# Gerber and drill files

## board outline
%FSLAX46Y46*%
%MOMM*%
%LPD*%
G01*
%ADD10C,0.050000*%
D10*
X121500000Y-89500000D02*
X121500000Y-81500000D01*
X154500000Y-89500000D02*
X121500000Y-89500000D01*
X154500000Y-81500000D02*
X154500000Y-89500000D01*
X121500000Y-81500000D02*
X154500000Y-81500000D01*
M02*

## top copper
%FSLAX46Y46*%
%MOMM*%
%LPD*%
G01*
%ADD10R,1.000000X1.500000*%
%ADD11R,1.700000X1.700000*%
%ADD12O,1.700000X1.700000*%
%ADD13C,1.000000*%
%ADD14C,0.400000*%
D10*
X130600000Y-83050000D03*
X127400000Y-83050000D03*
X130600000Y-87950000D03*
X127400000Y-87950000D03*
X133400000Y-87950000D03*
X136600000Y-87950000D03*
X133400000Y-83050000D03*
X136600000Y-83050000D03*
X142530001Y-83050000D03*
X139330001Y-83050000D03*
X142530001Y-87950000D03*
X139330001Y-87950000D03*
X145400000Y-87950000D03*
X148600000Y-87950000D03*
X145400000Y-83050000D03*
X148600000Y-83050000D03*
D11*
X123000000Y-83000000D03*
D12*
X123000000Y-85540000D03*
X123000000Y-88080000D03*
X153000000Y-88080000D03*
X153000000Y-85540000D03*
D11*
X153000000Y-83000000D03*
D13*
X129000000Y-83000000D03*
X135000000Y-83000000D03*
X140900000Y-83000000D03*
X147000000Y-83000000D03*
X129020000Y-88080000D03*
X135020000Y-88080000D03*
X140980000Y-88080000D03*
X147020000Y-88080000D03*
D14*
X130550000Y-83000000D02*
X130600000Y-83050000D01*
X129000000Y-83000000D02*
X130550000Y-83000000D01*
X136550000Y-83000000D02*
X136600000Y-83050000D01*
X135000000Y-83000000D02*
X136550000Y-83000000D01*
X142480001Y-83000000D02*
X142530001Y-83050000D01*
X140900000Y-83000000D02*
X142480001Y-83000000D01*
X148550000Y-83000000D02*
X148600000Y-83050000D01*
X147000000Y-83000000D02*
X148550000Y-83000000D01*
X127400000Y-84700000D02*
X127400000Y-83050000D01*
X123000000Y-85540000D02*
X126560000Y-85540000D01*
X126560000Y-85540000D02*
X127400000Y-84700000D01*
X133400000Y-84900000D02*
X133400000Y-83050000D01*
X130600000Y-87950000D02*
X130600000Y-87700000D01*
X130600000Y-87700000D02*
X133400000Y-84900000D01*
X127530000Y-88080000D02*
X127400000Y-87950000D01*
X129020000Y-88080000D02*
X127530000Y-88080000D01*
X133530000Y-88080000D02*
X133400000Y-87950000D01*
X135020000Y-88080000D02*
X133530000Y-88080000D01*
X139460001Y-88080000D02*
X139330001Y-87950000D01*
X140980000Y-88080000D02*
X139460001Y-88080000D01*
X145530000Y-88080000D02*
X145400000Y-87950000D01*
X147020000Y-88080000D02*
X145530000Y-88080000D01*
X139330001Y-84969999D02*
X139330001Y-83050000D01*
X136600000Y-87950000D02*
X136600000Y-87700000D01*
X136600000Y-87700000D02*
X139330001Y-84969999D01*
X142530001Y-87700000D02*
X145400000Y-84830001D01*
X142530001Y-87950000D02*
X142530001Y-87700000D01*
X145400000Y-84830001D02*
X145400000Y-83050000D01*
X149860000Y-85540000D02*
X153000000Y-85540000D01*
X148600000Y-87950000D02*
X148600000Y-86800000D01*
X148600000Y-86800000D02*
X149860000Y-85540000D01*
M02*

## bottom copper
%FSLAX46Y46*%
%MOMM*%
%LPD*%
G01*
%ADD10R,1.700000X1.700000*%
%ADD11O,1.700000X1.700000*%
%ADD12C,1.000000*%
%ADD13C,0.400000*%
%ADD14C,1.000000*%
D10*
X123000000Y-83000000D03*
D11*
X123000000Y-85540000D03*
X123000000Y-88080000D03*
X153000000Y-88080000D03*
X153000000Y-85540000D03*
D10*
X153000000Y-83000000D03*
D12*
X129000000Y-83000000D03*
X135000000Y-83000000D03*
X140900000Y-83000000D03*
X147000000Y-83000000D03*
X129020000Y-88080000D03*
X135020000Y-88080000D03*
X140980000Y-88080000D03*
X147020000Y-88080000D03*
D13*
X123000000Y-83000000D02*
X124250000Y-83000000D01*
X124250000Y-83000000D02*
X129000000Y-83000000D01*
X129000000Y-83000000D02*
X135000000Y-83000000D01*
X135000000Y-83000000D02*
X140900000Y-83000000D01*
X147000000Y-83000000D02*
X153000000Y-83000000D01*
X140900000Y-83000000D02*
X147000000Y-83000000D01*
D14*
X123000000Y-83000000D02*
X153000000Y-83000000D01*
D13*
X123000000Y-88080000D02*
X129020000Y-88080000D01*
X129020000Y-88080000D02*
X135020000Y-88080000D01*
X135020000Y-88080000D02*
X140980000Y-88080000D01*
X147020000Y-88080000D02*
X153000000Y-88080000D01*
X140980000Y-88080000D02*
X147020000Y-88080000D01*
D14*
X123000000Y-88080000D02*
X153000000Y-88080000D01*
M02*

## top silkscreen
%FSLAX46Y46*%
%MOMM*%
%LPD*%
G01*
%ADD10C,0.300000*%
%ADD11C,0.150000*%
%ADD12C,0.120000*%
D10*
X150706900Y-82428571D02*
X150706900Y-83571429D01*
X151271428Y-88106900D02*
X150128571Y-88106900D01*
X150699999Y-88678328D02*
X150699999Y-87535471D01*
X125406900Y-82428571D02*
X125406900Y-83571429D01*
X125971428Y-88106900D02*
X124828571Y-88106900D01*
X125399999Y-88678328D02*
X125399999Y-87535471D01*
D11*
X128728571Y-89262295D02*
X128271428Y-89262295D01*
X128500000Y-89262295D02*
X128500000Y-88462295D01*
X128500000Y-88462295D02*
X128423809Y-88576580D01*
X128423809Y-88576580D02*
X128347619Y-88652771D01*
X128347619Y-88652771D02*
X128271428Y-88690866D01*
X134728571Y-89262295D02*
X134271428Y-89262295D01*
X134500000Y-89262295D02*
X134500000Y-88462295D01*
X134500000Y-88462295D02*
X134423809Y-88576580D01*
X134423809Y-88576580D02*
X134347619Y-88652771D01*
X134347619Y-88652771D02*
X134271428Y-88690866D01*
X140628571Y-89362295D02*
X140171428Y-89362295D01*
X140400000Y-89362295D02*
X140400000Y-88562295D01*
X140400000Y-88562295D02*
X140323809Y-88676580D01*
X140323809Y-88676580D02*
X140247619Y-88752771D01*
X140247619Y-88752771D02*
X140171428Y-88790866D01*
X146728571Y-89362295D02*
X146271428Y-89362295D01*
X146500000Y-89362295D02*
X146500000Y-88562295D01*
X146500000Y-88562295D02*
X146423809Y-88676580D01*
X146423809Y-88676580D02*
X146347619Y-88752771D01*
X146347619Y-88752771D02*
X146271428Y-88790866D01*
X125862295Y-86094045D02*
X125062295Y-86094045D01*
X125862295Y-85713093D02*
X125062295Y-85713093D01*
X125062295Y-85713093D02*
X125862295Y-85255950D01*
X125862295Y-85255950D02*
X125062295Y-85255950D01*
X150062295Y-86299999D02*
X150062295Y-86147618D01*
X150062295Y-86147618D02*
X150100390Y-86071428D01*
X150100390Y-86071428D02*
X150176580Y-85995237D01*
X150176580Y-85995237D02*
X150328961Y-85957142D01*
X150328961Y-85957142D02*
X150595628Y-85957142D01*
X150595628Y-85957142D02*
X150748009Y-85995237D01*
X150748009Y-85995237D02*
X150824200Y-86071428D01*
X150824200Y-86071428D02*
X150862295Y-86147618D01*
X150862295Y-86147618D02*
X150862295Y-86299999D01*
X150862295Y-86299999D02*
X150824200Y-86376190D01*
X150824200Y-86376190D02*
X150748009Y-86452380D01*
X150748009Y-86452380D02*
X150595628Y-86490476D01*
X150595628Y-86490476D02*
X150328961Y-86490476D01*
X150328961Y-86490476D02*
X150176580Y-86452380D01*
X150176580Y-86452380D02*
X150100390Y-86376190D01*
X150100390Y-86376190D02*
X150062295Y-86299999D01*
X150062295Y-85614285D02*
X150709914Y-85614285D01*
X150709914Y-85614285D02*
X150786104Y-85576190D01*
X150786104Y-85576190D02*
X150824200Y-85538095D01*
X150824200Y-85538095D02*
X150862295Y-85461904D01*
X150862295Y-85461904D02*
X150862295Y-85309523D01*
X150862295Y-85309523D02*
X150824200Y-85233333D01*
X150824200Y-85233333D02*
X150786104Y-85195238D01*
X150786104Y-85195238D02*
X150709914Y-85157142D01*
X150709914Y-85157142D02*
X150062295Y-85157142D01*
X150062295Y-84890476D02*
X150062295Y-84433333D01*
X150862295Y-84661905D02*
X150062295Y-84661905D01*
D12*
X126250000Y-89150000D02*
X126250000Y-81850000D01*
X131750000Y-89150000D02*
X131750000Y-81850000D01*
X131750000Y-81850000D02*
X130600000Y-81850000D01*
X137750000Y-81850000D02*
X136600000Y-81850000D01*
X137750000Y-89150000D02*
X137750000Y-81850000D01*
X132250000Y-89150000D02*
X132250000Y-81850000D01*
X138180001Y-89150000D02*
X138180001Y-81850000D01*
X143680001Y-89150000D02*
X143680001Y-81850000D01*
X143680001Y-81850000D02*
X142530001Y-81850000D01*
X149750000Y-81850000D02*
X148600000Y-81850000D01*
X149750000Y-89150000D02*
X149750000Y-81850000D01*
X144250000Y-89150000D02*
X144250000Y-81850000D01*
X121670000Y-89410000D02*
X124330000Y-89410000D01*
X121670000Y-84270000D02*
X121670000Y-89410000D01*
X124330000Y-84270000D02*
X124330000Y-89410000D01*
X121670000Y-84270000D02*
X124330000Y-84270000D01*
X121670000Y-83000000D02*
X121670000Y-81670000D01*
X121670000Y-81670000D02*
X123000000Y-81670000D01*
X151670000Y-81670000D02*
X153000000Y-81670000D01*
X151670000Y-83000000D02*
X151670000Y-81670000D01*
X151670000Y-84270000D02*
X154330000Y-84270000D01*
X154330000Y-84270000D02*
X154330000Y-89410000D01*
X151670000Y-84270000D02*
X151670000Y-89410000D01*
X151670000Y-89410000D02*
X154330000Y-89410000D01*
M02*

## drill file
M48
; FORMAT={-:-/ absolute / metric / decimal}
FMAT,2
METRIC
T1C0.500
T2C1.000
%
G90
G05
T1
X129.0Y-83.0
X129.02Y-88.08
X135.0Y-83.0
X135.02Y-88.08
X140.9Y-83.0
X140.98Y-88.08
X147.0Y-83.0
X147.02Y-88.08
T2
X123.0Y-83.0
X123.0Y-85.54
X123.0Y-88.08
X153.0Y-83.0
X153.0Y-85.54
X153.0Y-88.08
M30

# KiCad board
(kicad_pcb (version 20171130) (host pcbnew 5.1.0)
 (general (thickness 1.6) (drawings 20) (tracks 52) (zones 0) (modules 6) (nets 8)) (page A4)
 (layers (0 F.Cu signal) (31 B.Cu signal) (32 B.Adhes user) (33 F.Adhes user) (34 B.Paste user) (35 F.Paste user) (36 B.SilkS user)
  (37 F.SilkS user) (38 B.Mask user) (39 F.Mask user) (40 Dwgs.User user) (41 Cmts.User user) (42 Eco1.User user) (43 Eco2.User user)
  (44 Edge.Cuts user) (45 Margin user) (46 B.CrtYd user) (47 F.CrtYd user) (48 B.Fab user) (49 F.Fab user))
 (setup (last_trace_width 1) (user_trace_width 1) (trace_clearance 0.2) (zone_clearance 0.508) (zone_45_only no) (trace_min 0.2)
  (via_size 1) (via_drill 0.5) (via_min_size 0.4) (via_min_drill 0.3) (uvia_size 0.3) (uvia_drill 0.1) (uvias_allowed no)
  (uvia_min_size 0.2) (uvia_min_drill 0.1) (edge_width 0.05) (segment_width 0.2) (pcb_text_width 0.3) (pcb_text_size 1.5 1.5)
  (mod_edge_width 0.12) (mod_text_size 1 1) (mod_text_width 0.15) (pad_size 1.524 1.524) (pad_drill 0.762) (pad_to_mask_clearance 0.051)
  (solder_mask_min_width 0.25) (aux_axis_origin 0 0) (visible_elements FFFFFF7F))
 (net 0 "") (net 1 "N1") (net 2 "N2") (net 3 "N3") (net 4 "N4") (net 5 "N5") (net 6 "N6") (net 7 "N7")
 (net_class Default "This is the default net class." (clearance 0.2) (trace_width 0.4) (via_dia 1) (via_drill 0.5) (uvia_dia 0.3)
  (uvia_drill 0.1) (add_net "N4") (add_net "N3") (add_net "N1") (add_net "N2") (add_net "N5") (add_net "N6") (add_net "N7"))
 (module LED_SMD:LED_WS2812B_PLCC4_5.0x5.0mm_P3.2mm (layer F.Cu) (at 129 85.5 90)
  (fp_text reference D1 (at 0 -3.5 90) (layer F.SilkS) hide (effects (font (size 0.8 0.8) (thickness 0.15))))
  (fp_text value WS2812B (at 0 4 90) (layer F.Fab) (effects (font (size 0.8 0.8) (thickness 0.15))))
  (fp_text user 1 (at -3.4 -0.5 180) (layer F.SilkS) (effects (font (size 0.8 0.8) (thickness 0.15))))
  (fp_line (start -3.65 -2.75) (end 3.65 -2.75) (layer F.SilkS) (width 0.12))
  (fp_line (start -3.65 2.75) (end 3.65 2.75) (layer F.SilkS) (width 0.12))
  (fp_line (start 3.65 2.75) (end 3.65 1.6) (layer F.SilkS) (width 0.12))
  (pad 3 smd rect (at 2.45 1.6 90) (size 1.5 1) (layers F.Cu F.Paste F.Mask) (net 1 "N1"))
  (pad 4 smd rect (at 2.45 -1.6 90) (size 1.5 1) (layers F.Cu F.Paste F.Mask) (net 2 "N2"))
  (pad 2 smd rect (at -2.45 1.6 90) (size 1.5 1) (layers F.Cu F.Paste F.Mask) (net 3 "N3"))
  (pad 1 smd rect (at -2.45 -1.6 90) (size 1.5 1) (layers F.Cu F.Paste F.Mask) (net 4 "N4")))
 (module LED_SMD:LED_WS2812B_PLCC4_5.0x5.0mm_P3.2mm (layer F.Cu) (at 135 85.5 90)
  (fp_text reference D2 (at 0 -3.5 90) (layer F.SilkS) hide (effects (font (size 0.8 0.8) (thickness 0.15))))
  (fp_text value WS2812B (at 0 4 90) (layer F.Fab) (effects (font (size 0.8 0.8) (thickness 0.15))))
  (fp_line (start 3.65 2.75) (end 3.65 1.6) (layer F.SilkS) (width 0.12))
  (fp_line (start -3.65 2.75) (end 3.65 2.75) (layer F.SilkS) (width 0.12))
  (fp_line (start -3.65 -2.75) (end 3.65 -2.75) (layer F.SilkS) (width 0.12))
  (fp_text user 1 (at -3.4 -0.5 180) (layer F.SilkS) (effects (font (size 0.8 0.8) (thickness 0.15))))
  (pad 1 smd rect (at -2.45 -1.6 90) (size 1.5 1) (layers F.Cu F.Paste F.Mask) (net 4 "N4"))
  (pad 2 smd rect (at -2.45 1.6 90) (size 1.5 1) (layers F.Cu F.Paste F.Mask) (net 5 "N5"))
  (pad 4 smd rect (at 2.45 -1.6 90) (size 1.5 1) (layers F.Cu F.Paste F.Mask) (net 3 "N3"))
  (pad 3 smd rect (at 2.45 1.6 90) (size 1.5 1) (layers F.Cu F.Paste F.Mask) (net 1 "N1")))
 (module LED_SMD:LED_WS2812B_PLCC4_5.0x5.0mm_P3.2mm (layer F.Cu) (at 140.930001 85.5 90)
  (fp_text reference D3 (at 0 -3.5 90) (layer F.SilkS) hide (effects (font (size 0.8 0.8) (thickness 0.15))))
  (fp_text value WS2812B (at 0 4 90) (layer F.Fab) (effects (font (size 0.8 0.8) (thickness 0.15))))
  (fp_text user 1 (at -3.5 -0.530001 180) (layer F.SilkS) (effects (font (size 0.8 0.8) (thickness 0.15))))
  (fp_line (start -3.65 -2.75) (end 3.65 -2.75) (layer F.SilkS) (width 0.12))
  (fp_line (start -3.65 2.75) (end 3.65 2.75) (layer F.SilkS) (width 0.12))
  (fp_line (start 3.65 2.75) (end 3.65 1.6) (layer F.SilkS) (width 0.12))
  (pad 3 smd rect (at 2.45 1.6 90) (size 1.5 1) (layers F.Cu F.Paste F.Mask) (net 1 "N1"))
  (pad 4 smd rect (at 2.45 -1.6 90) (size 1.5 1) (layers F.Cu F.Paste F.Mask) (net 5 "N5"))
  (pad 2 smd rect (at -2.45 1.6 90) (size 1.5 1) (layers F.Cu F.Paste F.Mask) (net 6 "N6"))
  (pad 1 smd rect (at -2.45 -1.6 90) (size 1.5 1) (layers F.Cu F.Paste F.Mask) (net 4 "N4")))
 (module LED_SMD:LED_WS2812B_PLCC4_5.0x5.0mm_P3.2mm (layer F.Cu) (at 147 85.5 90)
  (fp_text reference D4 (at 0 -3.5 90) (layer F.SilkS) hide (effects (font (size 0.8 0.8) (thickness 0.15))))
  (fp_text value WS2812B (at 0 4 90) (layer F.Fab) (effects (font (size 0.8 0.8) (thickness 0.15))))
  (fp_line (start 3.65 2.75) (end 3.65 1.6) (layer F.SilkS) (width 0.12))
  (fp_line (start -3.65 2.75) (end 3.65 2.75) (layer F.SilkS) (width 0.12))
  (fp_line (start -3.65 -2.75) (end 3.65 -2.75) (layer F.SilkS) (width 0.12))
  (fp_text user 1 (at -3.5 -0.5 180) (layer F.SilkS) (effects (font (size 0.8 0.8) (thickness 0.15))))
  (pad 1 smd rect (at -2.45 -1.6 90) (size 1.5 1) (layers F.Cu F.Paste F.Mask) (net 4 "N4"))
  (pad 2 smd rect (at -2.45 1.6 90) (size 1.5 1) (layers F.Cu F.Paste F.Mask) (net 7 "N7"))
  (pad 4 smd rect (at 2.45 -1.6 90) (size 1.5 1) (layers F.Cu F.Paste F.Mask) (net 6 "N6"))
  (pad 3 smd rect (at 2.45 1.6 90) (size 1.5 1) (layers F.Cu F.Paste F.Mask) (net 1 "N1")))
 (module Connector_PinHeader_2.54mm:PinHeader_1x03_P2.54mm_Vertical (layer F.Cu) (at 123 83)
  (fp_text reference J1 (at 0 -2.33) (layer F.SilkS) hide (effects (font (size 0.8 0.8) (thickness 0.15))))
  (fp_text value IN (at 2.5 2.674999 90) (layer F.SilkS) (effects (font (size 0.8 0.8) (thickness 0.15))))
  (fp_line (start -1.33 6.41) (end 1.33 6.41) (layer F.SilkS) (width 0.12))
  (fp_line (start -1.33 1.27) (end -1.33 6.41) (layer F.SilkS) (width 0.12))
  (fp_line (start 1.33 1.27) (end 1.33 6.41) (layer F.SilkS) (width 0.12))
  (fp_line (start -1.33 1.27) (end 1.33 1.27) (layer F.SilkS) (width 0.12))
  (fp_line (start -1.33 0) (end -1.33 -1.33) (layer F.SilkS) (width 0.12))
  (fp_line (start -1.33 -1.33) (end 0 -1.33) (layer F.SilkS) (width 0.12))
  (pad 1 thru_hole rect (at 0 0) (size 1.7 1.7) (drill 1) (layers *.Cu *.Mask) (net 1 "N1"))
  (pad 2 thru_hole oval (at 0 2.54) (size 1.7 1.7) (drill 1) (layers *.Cu *.Mask) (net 2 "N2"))
  (pad 3 thru_hole oval (at 0 5.08) (size 1.7 1.7) (drill 1) (layers *.Cu *.Mask) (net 4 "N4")))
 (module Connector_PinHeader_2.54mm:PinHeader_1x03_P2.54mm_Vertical (layer F.Cu) (at 153 83)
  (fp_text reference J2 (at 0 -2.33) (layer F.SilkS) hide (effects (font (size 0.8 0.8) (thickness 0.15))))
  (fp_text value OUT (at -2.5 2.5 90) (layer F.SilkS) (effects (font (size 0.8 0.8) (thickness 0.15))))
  (fp_line (start -1.33 -1.33) (end 0 -1.33) (layer F.SilkS) (width 0.12))
  (fp_line (start -1.33 0) (end -1.33 -1.33) (layer F.SilkS) (width 0.12))
  (fp_line (start -1.33 1.27) (end 1.33 1.27) (layer F.SilkS) (width 0.12))
  (fp_line (start 1.33 1.27) (end 1.33 6.41) (layer F.SilkS) (width 0.12))
  (fp_line (start -1.33 1.27) (end -1.33 6.41) (layer F.SilkS) (width 0.12))
  (fp_line (start -1.33 6.41) (end 1.33 6.41) (layer F.SilkS) (width 0.12))
  (pad 3 thru_hole oval (at 0 5.08) (size 1.7 1.7) (drill 1) (layers *.Cu *.Mask) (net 4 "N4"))
  (pad 2 thru_hole oval (at 0 2.54) (size 1.7 1.7) (drill 1) (layers *.Cu *.Mask) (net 7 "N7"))
  (pad 1 thru_hole rect (at 0 0) (size 1.7 1.7) (drill 1) (layers *.Cu *.Mask) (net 1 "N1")))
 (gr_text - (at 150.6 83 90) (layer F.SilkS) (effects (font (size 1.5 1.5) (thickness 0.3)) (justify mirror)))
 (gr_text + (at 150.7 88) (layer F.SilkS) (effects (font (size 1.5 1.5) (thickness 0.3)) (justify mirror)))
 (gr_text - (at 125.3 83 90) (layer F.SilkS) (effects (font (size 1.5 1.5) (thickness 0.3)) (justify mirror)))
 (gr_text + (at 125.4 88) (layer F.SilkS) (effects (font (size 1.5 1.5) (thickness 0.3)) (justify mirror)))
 (gr_line (start 121.5 89.5) (end 121.5 81.5) (layer Edge.Cuts) (width 0.05))
 (gr_line (start 154.5 89.5) (end 121.5 89.5) (layer Edge.Cuts) (width 0.05))
 (gr_line (start 154.5 81.5) (end 154.5 89.5) (layer Edge.Cuts) (width 0.05))
 (gr_line (start 121.5 81.5) (end 154.5 81.5) (layer Edge.Cuts) (width 0.05))
 (segment (start 123 83) (end 124.25 83) (width 0.4) (layer B.Cu) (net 1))
 (via (at 129 83) (size 1) (drill 0.5) (layers F.Cu B.Cu) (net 1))
 (segment (start 124.25 83) (end 129 83) (width 0.4) (layer B.Cu) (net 1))
 (segment (start 130.55 83) (end 130.6 83.05) (width 0.4) (layer F.Cu) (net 1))
 (segment (start 129 83) (end 130.55 83) (width 0.4) (layer F.Cu) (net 1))
 (via (at 135 83) (size 1) (drill 0.5) (layers F.Cu B.Cu) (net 1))
 (segment (start 129 83) (end 135 83) (width 0.4) (layer B.Cu) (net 1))
 (segment (start 136.55 83) (end 136.6 83.05) (width 0.4) (layer F.Cu) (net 1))
 (segment (start 135 83) (end 136.55 83) (width 0.4) (layer F.Cu) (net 1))
 (via (at 140.9 83) (size 1) (drill 0.5) (layers F.Cu B.Cu) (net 1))
 (segment (start 135 83) (end 140.9 83) (width 0.4) (layer B.Cu) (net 1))
 (segment (start 142.480001 83) (end 142.530001 83.05) (width 0.4) (layer F.Cu) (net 1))
 (segment (start 140.9 83) (end 142.480001 83) (width 0.4) (layer F.Cu) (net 1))
 (via (at 147 83) (size 1) (drill 0.5) (layers F.Cu B.Cu) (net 1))
 (segment (start 147 83) (end 153 83) (width 0.4) (layer B.Cu) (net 1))
 (segment (start 140.9 83) (end 147 83) (width 0.4) (layer B.Cu) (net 1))
 (segment (start 148.55 83) (end 148.6 83.05) (width 0.4) (layer F.Cu) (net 1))
 (segment (start 147 83) (end 148.55 83) (width 0.4) (layer F.Cu) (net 1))
 (segment (start 123 83) (end 153 83) (width 1) (layer B.Cu) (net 1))
 (segment (start 127.4 84.7) (end 127.4 83.05) (width 0.4) (layer F.Cu) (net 2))
 (segment (start 123 85.54) (end 126.56 85.54) (width 0.4) (layer F.Cu) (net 2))
 (segment (start 126.56 85.54) (end 127.4 84.7) (width 0.4) (layer F.Cu) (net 2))
 (segment (start 133.4 84.9) (end 133.4 83.05) (width 0.4) (layer F.Cu) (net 3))
 (segment (start 130.6 87.95) (end 130.6 87.7) (width 0.4) (layer F.Cu) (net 3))
 (segment (start 130.6 87.7) (end 133.4 84.9) (width 0.4) (layer F.Cu) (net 3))
 (via (at 129.02 88.08) (size 1) (drill 0.5) (layers F.Cu B.Cu) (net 4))
 (segment (start 123 88.08) (end 129.02 88.08) (width 0.4) (layer B.Cu) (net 4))
 (segment (start 127.53 88.08) (end 127.4 87.95) (width 0.4) (layer F.Cu) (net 4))
 (segment (start 129.02 88.08) (end 127.53 88.08) (width 0.4) (layer F.Cu) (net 4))
 (via (at 135.02 88.08) (size 1) (drill 0.5) (layers F.Cu B.Cu) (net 4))
 (segment (start 129.02 88.08) (end 135.02 88.08) (width 0.4) (layer B.Cu) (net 4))
 (segment (start 133.53 88.08) (end 133.4 87.95) (width 0.4) (layer F.Cu) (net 4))
 (segment (start 135.02 88.08) (end 133.53 88.08) (width 0.4) (layer F.Cu) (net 4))
 (via (at 140.98 88.08) (size 1) (drill 0.5) (layers F.Cu B.Cu) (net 4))
 (segment (start 135.02 88.08) (end 140.98 88.08) (width 0.4) (layer B.Cu) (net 4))
 (segment (start 139.460001 88.08) (end 139.330001 87.95) (width 0.4) (layer F.Cu) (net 4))
 (segment (start 140.98 88.08) (end 139.460001 88.08) (width 0.4) (layer F.Cu) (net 4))
 (via (at 147.02 88.08) (size 1) (drill 0.5) (layers F.Cu B.Cu) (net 4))
 (segment (start 147.02 88.08) (end 153 88.08) (width 0.4) (layer B.Cu) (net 4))
 (segment (start 140.98 88.08) (end 147.02 88.08) (width 0.4) (layer B.Cu) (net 4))
 (segment (start 145.53 88.08) (end 145.4 87.95) (width 0.4) (layer F.Cu) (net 4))
 (segment (start 147.02 88.08) (end 145.53 88.08) (width 0.4) (layer F.Cu) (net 4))
 (segment (start 123 88.08) (end 153 88.08) (width 1) (layer B.Cu) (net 4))
 (segment (start 139.330001 84.969999) (end 139.330001 83.05) (width 0.4) (layer F.Cu) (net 5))
 (segment (start 136.6 87.95) (end 136.6 87.7) (width 0.4) (layer F.Cu) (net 5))
 (segment (start 136.6 87.7) (end 139.330001 84.969999) (width 0.4) (layer F.Cu) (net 5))
 (segment (start 142.530001 87.7) (end 145.4 84.830001) (width 0.4) (layer F.Cu) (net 6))
 (segment (start 142.530001 87.95) (end 142.530001 87.7) (width 0.4) (layer F.Cu) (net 6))
 (segment (start 145.4 84.830001) (end 145.4 83.05) (width 0.4) (layer F.Cu) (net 6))
 (segment (start 149.86 85.54) (end 153 85.54) (width 0.4) (layer F.Cu) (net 7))
 (segment (start 148.6 87.95) (end 148.6 86.8) (width 0.4) (layer F.Cu) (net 7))
 (segment (start 148.6 86.8) (end 149.86 85.54) (width 0.4) (layer F.Cu) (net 7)))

